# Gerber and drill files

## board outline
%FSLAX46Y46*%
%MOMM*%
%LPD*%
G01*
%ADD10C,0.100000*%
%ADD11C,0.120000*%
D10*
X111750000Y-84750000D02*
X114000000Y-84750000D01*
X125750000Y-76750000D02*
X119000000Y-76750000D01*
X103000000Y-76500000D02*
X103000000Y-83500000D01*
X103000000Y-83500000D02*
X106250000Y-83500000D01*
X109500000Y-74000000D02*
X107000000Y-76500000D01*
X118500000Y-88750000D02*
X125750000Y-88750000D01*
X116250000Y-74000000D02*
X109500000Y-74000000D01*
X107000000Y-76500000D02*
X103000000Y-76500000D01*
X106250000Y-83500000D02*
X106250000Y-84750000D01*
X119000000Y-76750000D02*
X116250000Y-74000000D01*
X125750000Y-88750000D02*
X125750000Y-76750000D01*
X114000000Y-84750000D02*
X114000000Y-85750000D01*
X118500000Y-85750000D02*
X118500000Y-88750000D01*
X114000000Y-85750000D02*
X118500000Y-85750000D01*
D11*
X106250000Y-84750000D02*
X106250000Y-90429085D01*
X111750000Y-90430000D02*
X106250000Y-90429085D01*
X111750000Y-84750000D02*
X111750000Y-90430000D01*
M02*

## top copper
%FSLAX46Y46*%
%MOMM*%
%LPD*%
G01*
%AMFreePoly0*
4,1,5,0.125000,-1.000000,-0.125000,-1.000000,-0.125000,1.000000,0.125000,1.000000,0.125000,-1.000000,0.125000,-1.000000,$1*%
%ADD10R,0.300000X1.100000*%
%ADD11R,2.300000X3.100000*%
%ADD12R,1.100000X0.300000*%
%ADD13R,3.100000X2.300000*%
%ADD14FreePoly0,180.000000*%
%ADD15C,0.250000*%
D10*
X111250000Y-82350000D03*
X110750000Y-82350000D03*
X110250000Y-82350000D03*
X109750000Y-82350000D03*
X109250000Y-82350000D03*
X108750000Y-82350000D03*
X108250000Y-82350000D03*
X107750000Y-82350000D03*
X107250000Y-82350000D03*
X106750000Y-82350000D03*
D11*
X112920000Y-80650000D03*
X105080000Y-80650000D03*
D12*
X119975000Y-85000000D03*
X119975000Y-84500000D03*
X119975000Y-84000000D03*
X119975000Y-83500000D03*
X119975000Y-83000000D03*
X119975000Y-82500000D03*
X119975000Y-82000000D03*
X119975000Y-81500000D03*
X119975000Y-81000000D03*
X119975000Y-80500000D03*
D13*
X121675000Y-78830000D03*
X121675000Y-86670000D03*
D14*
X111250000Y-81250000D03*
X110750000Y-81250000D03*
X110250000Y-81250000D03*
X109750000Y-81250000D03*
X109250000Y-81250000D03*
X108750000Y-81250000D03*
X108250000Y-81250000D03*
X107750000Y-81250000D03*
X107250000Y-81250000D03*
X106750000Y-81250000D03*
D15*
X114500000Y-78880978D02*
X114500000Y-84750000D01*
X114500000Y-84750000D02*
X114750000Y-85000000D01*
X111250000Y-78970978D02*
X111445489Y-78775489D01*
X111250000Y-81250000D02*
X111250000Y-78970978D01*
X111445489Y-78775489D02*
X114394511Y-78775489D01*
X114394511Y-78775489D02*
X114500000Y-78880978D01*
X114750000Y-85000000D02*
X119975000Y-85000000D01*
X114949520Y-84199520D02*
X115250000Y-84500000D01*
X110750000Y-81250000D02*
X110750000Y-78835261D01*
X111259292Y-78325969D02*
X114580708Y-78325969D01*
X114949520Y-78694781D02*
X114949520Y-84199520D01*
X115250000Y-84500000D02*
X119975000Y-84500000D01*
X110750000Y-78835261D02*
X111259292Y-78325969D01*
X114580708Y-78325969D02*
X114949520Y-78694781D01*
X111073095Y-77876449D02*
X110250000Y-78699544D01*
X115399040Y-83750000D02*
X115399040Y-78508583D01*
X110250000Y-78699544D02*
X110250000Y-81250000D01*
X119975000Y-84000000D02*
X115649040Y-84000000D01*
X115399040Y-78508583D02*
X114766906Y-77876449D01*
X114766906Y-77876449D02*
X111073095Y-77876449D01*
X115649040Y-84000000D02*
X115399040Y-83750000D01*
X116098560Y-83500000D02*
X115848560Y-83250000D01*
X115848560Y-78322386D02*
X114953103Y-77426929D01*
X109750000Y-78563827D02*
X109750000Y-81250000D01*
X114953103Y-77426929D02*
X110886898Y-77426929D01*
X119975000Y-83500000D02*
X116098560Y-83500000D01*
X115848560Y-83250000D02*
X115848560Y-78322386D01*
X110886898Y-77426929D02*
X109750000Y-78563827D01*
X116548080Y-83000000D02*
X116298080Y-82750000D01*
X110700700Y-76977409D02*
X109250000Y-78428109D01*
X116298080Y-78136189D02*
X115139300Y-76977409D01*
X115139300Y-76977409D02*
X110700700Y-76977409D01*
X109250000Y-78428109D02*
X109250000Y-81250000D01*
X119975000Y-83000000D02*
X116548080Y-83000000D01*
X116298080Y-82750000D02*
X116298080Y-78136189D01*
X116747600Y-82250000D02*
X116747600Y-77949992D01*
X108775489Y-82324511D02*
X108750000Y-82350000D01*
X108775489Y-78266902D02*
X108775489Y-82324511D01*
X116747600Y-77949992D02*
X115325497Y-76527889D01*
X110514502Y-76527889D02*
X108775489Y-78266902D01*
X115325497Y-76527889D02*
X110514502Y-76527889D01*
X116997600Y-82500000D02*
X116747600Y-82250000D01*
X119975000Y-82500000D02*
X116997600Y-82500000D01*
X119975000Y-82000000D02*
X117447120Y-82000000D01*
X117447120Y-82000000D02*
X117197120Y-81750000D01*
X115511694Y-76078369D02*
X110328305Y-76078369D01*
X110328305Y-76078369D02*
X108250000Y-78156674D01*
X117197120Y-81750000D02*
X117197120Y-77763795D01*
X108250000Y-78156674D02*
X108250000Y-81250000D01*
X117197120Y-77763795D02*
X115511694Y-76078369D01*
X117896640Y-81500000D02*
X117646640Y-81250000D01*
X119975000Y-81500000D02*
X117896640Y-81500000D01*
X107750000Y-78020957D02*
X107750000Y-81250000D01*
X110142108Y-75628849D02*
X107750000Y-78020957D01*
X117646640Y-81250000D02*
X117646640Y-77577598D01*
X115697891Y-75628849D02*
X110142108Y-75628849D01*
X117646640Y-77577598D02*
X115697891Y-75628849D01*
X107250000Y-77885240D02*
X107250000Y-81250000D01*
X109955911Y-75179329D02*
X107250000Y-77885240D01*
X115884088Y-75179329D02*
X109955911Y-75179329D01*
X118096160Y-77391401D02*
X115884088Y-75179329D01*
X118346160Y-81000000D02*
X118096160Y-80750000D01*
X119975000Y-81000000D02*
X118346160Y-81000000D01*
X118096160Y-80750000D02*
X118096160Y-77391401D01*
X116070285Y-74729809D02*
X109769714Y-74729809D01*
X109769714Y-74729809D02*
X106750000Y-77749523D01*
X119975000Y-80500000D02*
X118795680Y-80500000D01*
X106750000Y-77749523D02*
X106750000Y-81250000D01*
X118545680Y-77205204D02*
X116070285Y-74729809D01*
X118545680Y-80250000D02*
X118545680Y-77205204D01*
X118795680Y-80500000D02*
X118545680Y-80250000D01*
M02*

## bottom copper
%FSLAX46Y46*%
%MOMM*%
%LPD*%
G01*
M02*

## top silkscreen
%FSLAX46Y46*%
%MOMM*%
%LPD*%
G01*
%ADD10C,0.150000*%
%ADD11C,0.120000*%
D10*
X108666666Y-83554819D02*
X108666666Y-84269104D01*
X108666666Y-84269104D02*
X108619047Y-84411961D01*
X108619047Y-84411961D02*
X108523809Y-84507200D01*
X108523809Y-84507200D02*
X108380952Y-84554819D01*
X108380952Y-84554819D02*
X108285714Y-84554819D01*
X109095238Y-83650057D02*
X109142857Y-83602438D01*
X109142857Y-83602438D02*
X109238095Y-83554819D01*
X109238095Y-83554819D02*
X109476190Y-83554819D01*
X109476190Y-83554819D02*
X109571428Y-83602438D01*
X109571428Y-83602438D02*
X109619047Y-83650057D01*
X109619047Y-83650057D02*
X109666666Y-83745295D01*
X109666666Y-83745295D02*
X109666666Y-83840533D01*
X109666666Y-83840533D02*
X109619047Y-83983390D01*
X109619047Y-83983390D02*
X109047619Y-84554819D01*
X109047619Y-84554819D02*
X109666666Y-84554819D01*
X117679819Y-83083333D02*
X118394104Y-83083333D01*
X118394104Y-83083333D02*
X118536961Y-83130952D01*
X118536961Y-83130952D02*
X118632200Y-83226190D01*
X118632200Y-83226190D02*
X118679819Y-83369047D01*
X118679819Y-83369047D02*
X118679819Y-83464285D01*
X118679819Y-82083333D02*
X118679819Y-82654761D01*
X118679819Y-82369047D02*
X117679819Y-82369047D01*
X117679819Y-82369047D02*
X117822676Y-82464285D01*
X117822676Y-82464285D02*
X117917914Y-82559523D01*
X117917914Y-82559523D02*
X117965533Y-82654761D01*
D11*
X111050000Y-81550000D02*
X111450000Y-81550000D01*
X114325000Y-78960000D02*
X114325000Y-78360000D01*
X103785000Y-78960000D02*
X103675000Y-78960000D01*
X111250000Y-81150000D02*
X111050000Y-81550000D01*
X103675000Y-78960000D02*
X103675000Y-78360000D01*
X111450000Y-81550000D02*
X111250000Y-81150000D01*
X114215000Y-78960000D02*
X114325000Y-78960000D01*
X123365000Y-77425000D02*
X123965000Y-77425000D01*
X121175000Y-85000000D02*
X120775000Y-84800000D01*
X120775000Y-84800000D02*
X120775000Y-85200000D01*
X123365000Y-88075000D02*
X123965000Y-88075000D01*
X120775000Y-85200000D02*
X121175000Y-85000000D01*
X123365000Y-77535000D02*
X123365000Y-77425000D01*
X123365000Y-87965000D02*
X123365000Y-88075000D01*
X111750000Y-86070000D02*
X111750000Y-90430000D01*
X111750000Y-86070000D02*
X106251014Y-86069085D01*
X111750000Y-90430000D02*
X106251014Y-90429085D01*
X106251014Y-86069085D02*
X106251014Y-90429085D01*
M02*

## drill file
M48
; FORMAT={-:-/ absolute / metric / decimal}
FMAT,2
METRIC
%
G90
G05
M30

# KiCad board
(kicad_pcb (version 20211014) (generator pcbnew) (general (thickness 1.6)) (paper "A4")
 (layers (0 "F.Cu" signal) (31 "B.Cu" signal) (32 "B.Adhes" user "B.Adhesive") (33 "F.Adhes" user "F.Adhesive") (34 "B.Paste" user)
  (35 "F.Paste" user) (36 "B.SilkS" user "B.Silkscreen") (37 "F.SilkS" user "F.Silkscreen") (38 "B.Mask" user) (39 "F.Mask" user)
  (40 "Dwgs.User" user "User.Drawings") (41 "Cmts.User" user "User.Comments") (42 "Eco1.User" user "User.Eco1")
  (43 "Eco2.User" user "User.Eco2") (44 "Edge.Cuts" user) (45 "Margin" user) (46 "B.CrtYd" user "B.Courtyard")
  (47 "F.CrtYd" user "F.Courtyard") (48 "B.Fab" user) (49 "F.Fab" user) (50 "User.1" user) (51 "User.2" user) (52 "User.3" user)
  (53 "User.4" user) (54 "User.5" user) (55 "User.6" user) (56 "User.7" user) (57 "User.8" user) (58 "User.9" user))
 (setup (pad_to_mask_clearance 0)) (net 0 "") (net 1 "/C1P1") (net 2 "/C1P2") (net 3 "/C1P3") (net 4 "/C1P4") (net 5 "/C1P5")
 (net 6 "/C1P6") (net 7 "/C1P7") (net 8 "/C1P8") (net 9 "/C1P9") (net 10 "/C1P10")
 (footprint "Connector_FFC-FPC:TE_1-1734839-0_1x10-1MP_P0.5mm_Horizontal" (layer "F.Cu") (at 109 81 180)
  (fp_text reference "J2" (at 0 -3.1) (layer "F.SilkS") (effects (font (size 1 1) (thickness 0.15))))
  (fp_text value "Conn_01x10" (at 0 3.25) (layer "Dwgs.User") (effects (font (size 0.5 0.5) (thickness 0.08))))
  (fp_line (start -2.05 -0.55) (end -2.45 -0.55) (layer "F.SilkS") (width 0.12))
  (fp_line (start -5.325 2.04) (end -5.325 2.64) (layer "F.SilkS") (width 0.12))
  (fp_line (start 5.215 2.04) (end 5.325 2.04) (layer "F.SilkS") (width 0.12))
  (fp_line (start -2.25 -0.15) (end -2.05 -0.55) (layer "F.SilkS") (width 0.12))
  (fp_line (start 5.325 2.04) (end 5.325 2.64) (layer "F.SilkS") (width 0.12))
  (fp_line (start -2.45 -0.55) (end -2.25 -0.15) (layer "F.SilkS") (width 0.12))
  (fp_line (start -5.215 2.04) (end -5.325 2.04) (layer "F.SilkS") (width 0.12))
  (pad "1" smd rect (at -2.25 -1.35 180) (size 0.3 1.1) (layers "F.Cu" "F.Paste" "F.Mask") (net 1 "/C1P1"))
  (pad "2" smd rect (at -1.75 -1.35 180) (size 0.3 1.1) (layers "F.Cu" "F.Paste" "F.Mask") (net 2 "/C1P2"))
  (pad "3" smd rect (at -1.25 -1.35 180) (size 0.3 1.1) (layers "F.Cu" "F.Paste" "F.Mask") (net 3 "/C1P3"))
  (pad "4" smd rect (at -0.75 -1.35 180) (size 0.3 1.1) (layers "F.Cu" "F.Paste" "F.Mask") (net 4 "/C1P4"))
  (pad "5" smd rect (at -0.25 -1.35 180) (size 0.3 1.1) (layers "F.Cu" "F.Paste" "F.Mask") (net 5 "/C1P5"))
  (pad "6" smd rect (at 0.25 -1.35 180) (size 0.3 1.1) (layers "F.Cu" "F.Paste" "F.Mask") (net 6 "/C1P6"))
  (pad "7" smd rect (at 0.75 -1.35 180) (size 0.3 1.1) (layers "F.Cu" "F.Paste" "F.Mask") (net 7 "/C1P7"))
  (pad "8" smd rect (at 1.25 -1.35 180) (size 0.3 1.1) (layers "F.Cu" "F.Paste" "F.Mask") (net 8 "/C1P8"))
  (pad "9" smd rect (at 1.75 -1.35 180) (size 0.3 1.1) (layers "F.Cu" "F.Paste" "F.Mask") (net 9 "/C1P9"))
  (pad "10" smd rect (at 2.25 -1.35 180) (size 0.3 1.1) (layers "F.Cu" "F.Paste" "F.Mask") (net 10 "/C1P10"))
  (pad "MP" smd rect (at -3.92 0.35 180) (size 2.3 3.1) (layers "F.Cu" "F.Paste" "F.Mask"))
  (pad "MP" smd rect (at 3.92 0.35 180) (size 2.3 3.1) (layers "F.Cu" "F.Paste" "F.Mask")))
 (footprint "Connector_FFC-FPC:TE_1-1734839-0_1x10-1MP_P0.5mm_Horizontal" (layer "F.Cu") (at 121.325 82.75 90)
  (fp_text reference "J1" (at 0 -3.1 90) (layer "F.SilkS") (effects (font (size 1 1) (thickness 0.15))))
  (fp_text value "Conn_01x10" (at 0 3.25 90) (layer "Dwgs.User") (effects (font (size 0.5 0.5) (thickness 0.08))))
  (fp_line (start 5.325 2.04) (end 5.325 2.64) (layer "F.SilkS") (width 0.12))
  (fp_line (start -2.25 -0.15) (end -2.05 -0.55) (layer "F.SilkS") (width 0.12))
  (fp_line (start -2.05 -0.55) (end -2.45 -0.55) (layer "F.SilkS") (width 0.12))
  (fp_line (start -5.325 2.04) (end -5.325 2.64) (layer "F.SilkS") (width 0.12))
  (fp_line (start -2.45 -0.55) (end -2.25 -0.15) (layer "F.SilkS") (width 0.12))
  (fp_line (start 5.215 2.04) (end 5.325 2.04) (layer "F.SilkS") (width 0.12))
  (fp_line (start -5.215 2.04) (end -5.325 2.04) (layer "F.SilkS") (width 0.12))
  (pad "1" smd rect (at -2.25 -1.35 90) (size 0.3 1.1) (layers "F.Cu" "F.Paste" "F.Mask") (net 1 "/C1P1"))
  (pad "2" smd rect (at -1.75 -1.35 90) (size 0.3 1.1) (layers "F.Cu" "F.Paste" "F.Mask") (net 2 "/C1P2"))
  (pad "3" smd rect (at -1.25 -1.35 90) (size 0.3 1.1) (layers "F.Cu" "F.Paste" "F.Mask") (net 3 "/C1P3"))
  (pad "4" smd rect (at -0.75 -1.35 90) (size 0.3 1.1) (layers "F.Cu" "F.Paste" "F.Mask") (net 4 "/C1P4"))
  (pad "5" smd rect (at -0.25 -1.35 90) (size 0.3 1.1) (layers "F.Cu" "F.Paste" "F.Mask") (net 5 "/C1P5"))
  (pad "6" smd rect (at 0.25 -1.35 90) (size 0.3 1.1) (layers "F.Cu" "F.Paste" "F.Mask") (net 6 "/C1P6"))
  (pad "7" smd rect (at 0.75 -1.35 90) (size 0.3 1.1) (layers "F.Cu" "F.Paste" "F.Mask") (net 7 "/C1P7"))
  (pad "8" smd rect (at 1.25 -1.35 90) (size 0.3 1.1) (layers "F.Cu" "F.Paste" "F.Mask") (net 8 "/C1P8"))
  (pad "9" smd rect (at 1.75 -1.35 90) (size 0.3 1.1) (layers "F.Cu" "F.Paste" "F.Mask") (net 9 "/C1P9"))
  (pad "10" smd rect (at 2.25 -1.35 90) (size 0.3 1.1) (layers "F.Cu" "F.Paste" "F.Mask") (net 10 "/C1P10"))
  (pad "MP" smd rect (at 3.92 0.35 90) (size 2.3 3.1) (layers "F.Cu" "F.Paste" "F.Mask"))
  (pad "MP" smd rect (at -3.92 0.35 90) (size 2.3 3.1) (layers "F.Cu" "F.Paste" "F.Mask")))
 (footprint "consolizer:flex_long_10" (layer "F.Cu") (at 108.75 86.25 180)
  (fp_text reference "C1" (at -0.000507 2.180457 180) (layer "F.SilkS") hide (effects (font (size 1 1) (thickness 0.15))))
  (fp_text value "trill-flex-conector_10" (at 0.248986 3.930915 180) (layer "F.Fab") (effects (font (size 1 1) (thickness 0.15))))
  (fp_line (start -3 0.18) (end -3 -4.18) (layer "F.SilkS") (width 0.12))
  (fp_line (start -3 0.18) (end 2.498986 0.180915) (layer "F.SilkS") (width 0.12))
  (fp_line (start -3 -4.18) (end 2.498986 -4.179085) (layer "F.SilkS") (width 0.12))
  (fp_line (start 2.498986 0.180915) (end 2.498986 -4.179085) (layer "F.SilkS") (width 0.12))
  (fp_line (start 2.5 1.5) (end 2.5 -4.179085) (layer "Edge.Cuts") (width 0.12))
  (fp_line (start -3 -4.18) (end 2.5 -4.179085) (layer "Edge.Cuts") (width 0.12))
  (fp_line (start -3 1.5) (end -3 -4.18) (layer "Edge.Cuts") (width 0.12))
  (pad "" smd rect (at 1.5 -2 180) (size 0.25 4) (layers "F.Paste" "F.Mask"))
  (pad "" smd rect (at -0.5 -2 180) (size 0.25 4) (layers "F.Paste" "F.Mask"))
  (pad "" smd rect (at -2.5 -2 180) (size 0.25 4) (layers "F.Paste" "F.Mask"))
  (pad "" smd rect (at 0.5 -2 180) (size 0.25 4) (layers "F.Paste" "F.Mask"))
  (pad "" smd rect (at -1 -2 180) (size 0.25 4) (layers "F.Paste" "F.Mask"))
  (pad "" smd rect (at 1 -2 180) (size 0.25 4) (layers "F.Paste" "F.Mask"))
  (pad "" smd rect (at 1.998986 -1.999085 180) (size 0.25 4) (layers "F.Paste" "F.Mask"))
  (pad "" smd rect (at -1.5 -2 180) (size 0.25 4) (layers "F.Paste" "F.Mask"))
  (pad "" smd rect (at 0 -2 180) (size 0.25 4) (layers "F.Paste" "F.Mask"))
  (pad "" smd rect (at -2 -2 180) (size 0.25 4) (layers "F.Paste" "F.Mask"))
  (pad "1" smd custom (at -2.5 5 180) (size 0.25 2) (layers "F.Cu") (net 1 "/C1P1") (zone_connect 0)
   (options (clearance outline) (anchor rect)) (primitives))
  (pad "2" smd custom (at -2 5 180) (size 0.25 2) (layers "F.Cu") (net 2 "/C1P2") (zone_connect 0)
   (options (clearance outline) (anchor rect)) (primitives))
  (pad "3" smd custom (at -1.5 5 180) (size 0.25 2) (layers "F.Cu") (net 3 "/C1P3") (zone_connect 0)
   (options (clearance outline) (anchor rect)) (primitives))
  (pad "4" smd custom (at -1 5 180) (size 0.25 2) (layers "F.Cu") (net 4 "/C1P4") (zone_connect 0)
   (options (clearance outline) (anchor rect)) (primitives))
  (pad "5" smd custom (at -0.5 5 180) (size 0.25 2) (layers "F.Cu") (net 5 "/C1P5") (zone_connect 0)
   (options (clearance outline) (anchor rect)) (primitives))
  (pad "6" smd custom (at 0 5 180) (size 0.25 2) (layers "F.Cu") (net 6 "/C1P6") (zone_connect 0)
   (options (clearance outline) (anchor rect)) (primitives))
  (pad "7" smd custom (at 0.5 5 180) (size 0.25 2) (layers "F.Cu") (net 7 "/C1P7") (zone_connect 0)
   (options (clearance outline) (anchor rect)) (primitives))
  (pad "8" smd custom (at 1 5 180) (size 0.25 2) (layers "F.Cu") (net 8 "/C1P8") (zone_connect 0)
   (options (clearance outline) (anchor rect)) (primitives))
  (pad "9" smd custom (at 1.5 5 180) (size 0.25 2) (layers "F.Cu") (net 9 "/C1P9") (zone_connect 0)
   (options (clearance outline) (anchor rect)) (primitives))
  (pad "10" smd custom (at 2 5 180) (size 0.25 2) (layers "F.Cu") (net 10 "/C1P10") (zone_connect 0)
   (options (clearance outline) (anchor rect)) (primitives)))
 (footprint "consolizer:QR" (layer "B.Cu") (at 113 79 180)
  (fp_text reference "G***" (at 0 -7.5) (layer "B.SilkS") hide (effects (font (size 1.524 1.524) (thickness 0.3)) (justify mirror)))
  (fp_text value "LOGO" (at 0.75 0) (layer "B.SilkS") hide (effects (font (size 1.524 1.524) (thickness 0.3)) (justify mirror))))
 (gr_line (start 111.75 84.75) (end 114 84.75) (layer "Edge.Cuts") (width 0.1))
 (gr_line (start 125.75 76.75) (end 119 76.75) (layer "Edge.Cuts") (width 0.1))
 (gr_line (start 103 76.5) (end 103 83.5) (layer "Edge.Cuts") (width 0.1))
 (gr_line (start 103 83.5) (end 106.25 83.5) (layer "Edge.Cuts") (width 0.1))
 (gr_line (start 109.5 74) (end 107 76.5) (layer "Edge.Cuts") (width 0.1))
 (gr_line (start 118.5 88.75) (end 125.75 88.75) (layer "Edge.Cuts") (width 0.1))
 (gr_line (start 116.25 74) (end 109.5 74) (layer "Edge.Cuts") (width 0.1))
 (gr_line (start 107 76.5) (end 103 76.5) (layer "Edge.Cuts") (width 0.1))
 (gr_line (start 106.25 83.5) (end 106.25 84.75) (layer "Edge.Cuts") (width 0.1))
 (gr_line (start 119 76.75) (end 116.25 74) (layer "Edge.Cuts") (width 0.1))
 (gr_line (start 125.75 88.75) (end 125.75 76.75) (layer "Edge.Cuts") (width 0.1))
 (gr_line (start 114 84.75) (end 114 85.75) (layer "Edge.Cuts") (width 0.1))
 (gr_line (start 118.5 85.75) (end 118.5 88.75) (layer "Edge.Cuts") (width 0.1))
 (gr_line (start 114 85.75) (end 118.5 85.75) (layer "Edge.Cuts") (width 0.1))
 (segment (start 114.5 78.880978) (end 114.5 84.75) (width 0.25) (layer "F.Cu") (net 1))
 (segment (start 114.5 84.75) (end 114.75 85) (width 0.25) (layer "F.Cu") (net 1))
 (segment (start 111.25 78.970978) (end 111.445489 78.775489) (width 0.25) (layer "F.Cu") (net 1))
 (segment (start 111.25 81.25) (end 111.25 78.970978) (width 0.25) (layer "F.Cu") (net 1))
 (segment (start 111.445489 78.775489) (end 114.394511 78.775489) (width 0.25) (layer "F.Cu") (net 1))
 (segment (start 114.394511 78.775489) (end 114.5 78.880978) (width 0.25) (layer "F.Cu") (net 1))
 (segment (start 114.75 85) (end 119.975 85) (width 0.25) (layer "F.Cu") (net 1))
 (segment (start 114.94952 84.19952) (end 115.25 84.5) (width 0.25) (layer "F.Cu") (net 2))
 (segment (start 110.75 81.25) (end 110.75 78.835261) (width 0.25) (layer "F.Cu") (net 2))
 (segment (start 111.259292 78.325969) (end 114.580708 78.325969) (width 0.25) (layer "F.Cu") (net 2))
 (segment (start 114.94952 78.694781) (end 114.94952 84.19952) (width 0.25) (layer "F.Cu") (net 2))
 (segment (start 115.25 84.5) (end 119.975 84.5) (width 0.25) (layer "F.Cu") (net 2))
 (segment (start 110.75 78.835261) (end 111.259292 78.325969) (width 0.25) (layer "F.Cu") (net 2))
 (segment (start 114.580708 78.325969) (end 114.94952 78.694781) (width 0.25) (layer "F.Cu") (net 2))
 (segment (start 111.073095 77.876449) (end 110.25 78.699544) (width 0.25) (layer "F.Cu") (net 3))
 (segment (start 115.39904 83.75) (end 115.39904 78.508583) (width 0.25) (layer "F.Cu") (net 3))
 (segment (start 110.25 78.699544) (end 110.25 81.25) (width 0.25) (layer "F.Cu") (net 3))
 (segment (start 119.975 84) (end 115.64904 84) (width 0.25) (layer "F.Cu") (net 3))
 (segment (start 115.39904 78.508583) (end 114.766906 77.876449) (width 0.25) (layer "F.Cu") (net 3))
 (segment (start 114.766906 77.876449) (end 111.073095 77.876449) (width 0.25) (layer "F.Cu") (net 3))
 (segment (start 115.64904 84) (end 115.39904 83.75) (width 0.25) (layer "F.Cu") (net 3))
 (segment (start 116.09856 83.5) (end 115.84856 83.25) (width 0.25) (layer "F.Cu") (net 4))
 (segment (start 115.84856 78.322386) (end 114.953103 77.426929) (width 0.25) (layer "F.Cu") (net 4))
 (segment (start 109.75 78.563827) (end 109.75 81.25) (width 0.25) (layer "F.Cu") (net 4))
 (segment (start 114.953103 77.426929) (end 110.886898 77.426929) (width 0.25) (layer "F.Cu") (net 4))
 (segment (start 119.975 83.5) (end 116.09856 83.5) (width 0.25) (layer "F.Cu") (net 4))
 (segment (start 115.84856 83.25) (end 115.84856 78.322386) (width 0.25) (layer "F.Cu") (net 4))
 (segment (start 110.886898 77.426929) (end 109.75 78.563827) (width 0.25) (layer "F.Cu") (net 4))
 (segment (start 116.54808 83) (end 116.29808 82.75) (width 0.25) (layer "F.Cu") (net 5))
 (segment (start 110.7007 76.977409) (end 109.25 78.428109) (width 0.25) (layer "F.Cu") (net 5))
 (segment (start 116.29808 78.136189) (end 115.1393 76.977409) (width 0.25) (layer "F.Cu") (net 5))
 (segment (start 115.1393 76.977409) (end 110.7007 76.977409) (width 0.25) (layer "F.Cu") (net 5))
 (segment (start 109.25 78.428109) (end 109.25 81.25) (width 0.25) (layer "F.Cu") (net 5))
 (segment (start 119.975 83) (end 116.54808 83) (width 0.25) (layer "F.Cu") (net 5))
 (segment (start 116.29808 82.75) (end 116.29808 78.136189) (width 0.25) (layer "F.Cu") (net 5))
 (segment (start 116.7476 82.25) (end 116.7476 77.949992) (width 0.25) (layer "F.Cu") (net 6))
 (segment (start 108.775489 82.324511) (end 108.75 82.35) (width 0.25) (layer "F.Cu") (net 6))
 (segment (start 108.775489 78.266902) (end 108.775489 82.324511) (width 0.25) (layer "F.Cu") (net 6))
 (segment (start 116.7476 77.949992) (end 115.325497 76.527889) (width 0.25) (layer "F.Cu") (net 6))
 (segment (start 110.514502 76.527889) (end 108.775489 78.266902) (width 0.25) (layer "F.Cu") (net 6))
 (segment (start 115.325497 76.527889) (end 110.514502 76.527889) (width 0.25) (layer "F.Cu") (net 6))
 (segment (start 116.9976 82.5) (end 116.7476 82.25) (width 0.25) (layer "F.Cu") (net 6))
 (segment (start 119.975 82.5) (end 116.9976 82.5) (width 0.25) (layer "F.Cu") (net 6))
 (segment (start 119.975 82) (end 117.44712 82) (width 0.25) (layer "F.Cu") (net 7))
 (segment (start 117.44712 82) (end 117.19712 81.75) (width 0.25) (layer "F.Cu") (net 7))
 (segment (start 115.511694 76.078369) (end 110.328305 76.078369) (width 0.25) (layer "F.Cu") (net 7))
 (segment (start 110.328305 76.078369) (end 108.25 78.156674) (width 0.25) (layer "F.Cu") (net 7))
 (segment (start 117.19712 81.75) (end 117.19712 77.763795) (width 0.25) (layer "F.Cu") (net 7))
 (segment (start 108.25 78.156674) (end 108.25 81.25) (width 0.25) (layer "F.Cu") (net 7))
 (segment (start 117.19712 77.763795) (end 115.511694 76.078369) (width 0.25) (layer "F.Cu") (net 7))
 (segment (start 117.89664 81.5) (end 117.64664 81.25) (width 0.25) (layer "F.Cu") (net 8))
 (segment (start 119.975 81.5) (end 117.89664 81.5) (width 0.25) (layer "F.Cu") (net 8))
 (segment (start 107.75 78.020957) (end 107.75 81.25) (width 0.25) (layer "F.Cu") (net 8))
 (segment (start 110.142108 75.628849) (end 107.75 78.020957) (width 0.25) (layer "F.Cu") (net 8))
 (segment (start 117.64664 81.25) (end 117.64664 77.577598) (width 0.25) (layer "F.Cu") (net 8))
 (segment (start 115.697891 75.628849) (end 110.142108 75.628849) (width 0.25) (layer "F.Cu") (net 8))
 (segment (start 117.64664 77.577598) (end 115.697891 75.628849) (width 0.25) (layer "F.Cu") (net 8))
 (segment (start 107.25 77.88524) (end 107.25 81.25) (width 0.25) (layer "F.Cu") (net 9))
 (segment (start 109.955911 75.179329) (end 107.25 77.88524) (width 0.25) (layer "F.Cu") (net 9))
 (segment (start 115.884088 75.179329) (end 109.955911 75.179329) (width 0.25) (layer "F.Cu") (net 9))
 (segment (start 118.09616 77.391401) (end 115.884088 75.179329) (width 0.25) (layer "F.Cu") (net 9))
 (segment (start 118.34616 81) (end 118.09616 80.75) (width 0.25) (layer "F.Cu") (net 9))
 (segment (start 119.975 81) (end 118.34616 81) (width 0.25) (layer "F.Cu") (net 9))
 (segment (start 118.09616 80.75) (end 118.09616 77.391401) (width 0.25) (layer "F.Cu") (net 9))
 (segment (start 116.070285 74.729809) (end 109.769714 74.729809) (width 0.25) (layer "F.Cu") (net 10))
 (segment (start 109.769714 74.729809) (end 106.75 77.749523) (width 0.25) (layer "F.Cu") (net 10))
 (segment (start 119.975 80.5) (end 118.79568 80.5) (width 0.25) (layer "F.Cu") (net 10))
 (segment (start 106.75 77.749523) (end 106.75 81.25) (width 0.25) (layer "F.Cu") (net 10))
 (segment (start 118.54568 77.205204) (end 116.070285 74.729809) (width 0.25) (layer "F.Cu") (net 10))
 (segment (start 118.54568 80.25) (end 118.54568 77.205204) (width 0.25) (layer "F.Cu") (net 10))
 (segment (start 118.79568 80.5) (end 118.54568 80.25) (width 0.25) (layer "F.Cu") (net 10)))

